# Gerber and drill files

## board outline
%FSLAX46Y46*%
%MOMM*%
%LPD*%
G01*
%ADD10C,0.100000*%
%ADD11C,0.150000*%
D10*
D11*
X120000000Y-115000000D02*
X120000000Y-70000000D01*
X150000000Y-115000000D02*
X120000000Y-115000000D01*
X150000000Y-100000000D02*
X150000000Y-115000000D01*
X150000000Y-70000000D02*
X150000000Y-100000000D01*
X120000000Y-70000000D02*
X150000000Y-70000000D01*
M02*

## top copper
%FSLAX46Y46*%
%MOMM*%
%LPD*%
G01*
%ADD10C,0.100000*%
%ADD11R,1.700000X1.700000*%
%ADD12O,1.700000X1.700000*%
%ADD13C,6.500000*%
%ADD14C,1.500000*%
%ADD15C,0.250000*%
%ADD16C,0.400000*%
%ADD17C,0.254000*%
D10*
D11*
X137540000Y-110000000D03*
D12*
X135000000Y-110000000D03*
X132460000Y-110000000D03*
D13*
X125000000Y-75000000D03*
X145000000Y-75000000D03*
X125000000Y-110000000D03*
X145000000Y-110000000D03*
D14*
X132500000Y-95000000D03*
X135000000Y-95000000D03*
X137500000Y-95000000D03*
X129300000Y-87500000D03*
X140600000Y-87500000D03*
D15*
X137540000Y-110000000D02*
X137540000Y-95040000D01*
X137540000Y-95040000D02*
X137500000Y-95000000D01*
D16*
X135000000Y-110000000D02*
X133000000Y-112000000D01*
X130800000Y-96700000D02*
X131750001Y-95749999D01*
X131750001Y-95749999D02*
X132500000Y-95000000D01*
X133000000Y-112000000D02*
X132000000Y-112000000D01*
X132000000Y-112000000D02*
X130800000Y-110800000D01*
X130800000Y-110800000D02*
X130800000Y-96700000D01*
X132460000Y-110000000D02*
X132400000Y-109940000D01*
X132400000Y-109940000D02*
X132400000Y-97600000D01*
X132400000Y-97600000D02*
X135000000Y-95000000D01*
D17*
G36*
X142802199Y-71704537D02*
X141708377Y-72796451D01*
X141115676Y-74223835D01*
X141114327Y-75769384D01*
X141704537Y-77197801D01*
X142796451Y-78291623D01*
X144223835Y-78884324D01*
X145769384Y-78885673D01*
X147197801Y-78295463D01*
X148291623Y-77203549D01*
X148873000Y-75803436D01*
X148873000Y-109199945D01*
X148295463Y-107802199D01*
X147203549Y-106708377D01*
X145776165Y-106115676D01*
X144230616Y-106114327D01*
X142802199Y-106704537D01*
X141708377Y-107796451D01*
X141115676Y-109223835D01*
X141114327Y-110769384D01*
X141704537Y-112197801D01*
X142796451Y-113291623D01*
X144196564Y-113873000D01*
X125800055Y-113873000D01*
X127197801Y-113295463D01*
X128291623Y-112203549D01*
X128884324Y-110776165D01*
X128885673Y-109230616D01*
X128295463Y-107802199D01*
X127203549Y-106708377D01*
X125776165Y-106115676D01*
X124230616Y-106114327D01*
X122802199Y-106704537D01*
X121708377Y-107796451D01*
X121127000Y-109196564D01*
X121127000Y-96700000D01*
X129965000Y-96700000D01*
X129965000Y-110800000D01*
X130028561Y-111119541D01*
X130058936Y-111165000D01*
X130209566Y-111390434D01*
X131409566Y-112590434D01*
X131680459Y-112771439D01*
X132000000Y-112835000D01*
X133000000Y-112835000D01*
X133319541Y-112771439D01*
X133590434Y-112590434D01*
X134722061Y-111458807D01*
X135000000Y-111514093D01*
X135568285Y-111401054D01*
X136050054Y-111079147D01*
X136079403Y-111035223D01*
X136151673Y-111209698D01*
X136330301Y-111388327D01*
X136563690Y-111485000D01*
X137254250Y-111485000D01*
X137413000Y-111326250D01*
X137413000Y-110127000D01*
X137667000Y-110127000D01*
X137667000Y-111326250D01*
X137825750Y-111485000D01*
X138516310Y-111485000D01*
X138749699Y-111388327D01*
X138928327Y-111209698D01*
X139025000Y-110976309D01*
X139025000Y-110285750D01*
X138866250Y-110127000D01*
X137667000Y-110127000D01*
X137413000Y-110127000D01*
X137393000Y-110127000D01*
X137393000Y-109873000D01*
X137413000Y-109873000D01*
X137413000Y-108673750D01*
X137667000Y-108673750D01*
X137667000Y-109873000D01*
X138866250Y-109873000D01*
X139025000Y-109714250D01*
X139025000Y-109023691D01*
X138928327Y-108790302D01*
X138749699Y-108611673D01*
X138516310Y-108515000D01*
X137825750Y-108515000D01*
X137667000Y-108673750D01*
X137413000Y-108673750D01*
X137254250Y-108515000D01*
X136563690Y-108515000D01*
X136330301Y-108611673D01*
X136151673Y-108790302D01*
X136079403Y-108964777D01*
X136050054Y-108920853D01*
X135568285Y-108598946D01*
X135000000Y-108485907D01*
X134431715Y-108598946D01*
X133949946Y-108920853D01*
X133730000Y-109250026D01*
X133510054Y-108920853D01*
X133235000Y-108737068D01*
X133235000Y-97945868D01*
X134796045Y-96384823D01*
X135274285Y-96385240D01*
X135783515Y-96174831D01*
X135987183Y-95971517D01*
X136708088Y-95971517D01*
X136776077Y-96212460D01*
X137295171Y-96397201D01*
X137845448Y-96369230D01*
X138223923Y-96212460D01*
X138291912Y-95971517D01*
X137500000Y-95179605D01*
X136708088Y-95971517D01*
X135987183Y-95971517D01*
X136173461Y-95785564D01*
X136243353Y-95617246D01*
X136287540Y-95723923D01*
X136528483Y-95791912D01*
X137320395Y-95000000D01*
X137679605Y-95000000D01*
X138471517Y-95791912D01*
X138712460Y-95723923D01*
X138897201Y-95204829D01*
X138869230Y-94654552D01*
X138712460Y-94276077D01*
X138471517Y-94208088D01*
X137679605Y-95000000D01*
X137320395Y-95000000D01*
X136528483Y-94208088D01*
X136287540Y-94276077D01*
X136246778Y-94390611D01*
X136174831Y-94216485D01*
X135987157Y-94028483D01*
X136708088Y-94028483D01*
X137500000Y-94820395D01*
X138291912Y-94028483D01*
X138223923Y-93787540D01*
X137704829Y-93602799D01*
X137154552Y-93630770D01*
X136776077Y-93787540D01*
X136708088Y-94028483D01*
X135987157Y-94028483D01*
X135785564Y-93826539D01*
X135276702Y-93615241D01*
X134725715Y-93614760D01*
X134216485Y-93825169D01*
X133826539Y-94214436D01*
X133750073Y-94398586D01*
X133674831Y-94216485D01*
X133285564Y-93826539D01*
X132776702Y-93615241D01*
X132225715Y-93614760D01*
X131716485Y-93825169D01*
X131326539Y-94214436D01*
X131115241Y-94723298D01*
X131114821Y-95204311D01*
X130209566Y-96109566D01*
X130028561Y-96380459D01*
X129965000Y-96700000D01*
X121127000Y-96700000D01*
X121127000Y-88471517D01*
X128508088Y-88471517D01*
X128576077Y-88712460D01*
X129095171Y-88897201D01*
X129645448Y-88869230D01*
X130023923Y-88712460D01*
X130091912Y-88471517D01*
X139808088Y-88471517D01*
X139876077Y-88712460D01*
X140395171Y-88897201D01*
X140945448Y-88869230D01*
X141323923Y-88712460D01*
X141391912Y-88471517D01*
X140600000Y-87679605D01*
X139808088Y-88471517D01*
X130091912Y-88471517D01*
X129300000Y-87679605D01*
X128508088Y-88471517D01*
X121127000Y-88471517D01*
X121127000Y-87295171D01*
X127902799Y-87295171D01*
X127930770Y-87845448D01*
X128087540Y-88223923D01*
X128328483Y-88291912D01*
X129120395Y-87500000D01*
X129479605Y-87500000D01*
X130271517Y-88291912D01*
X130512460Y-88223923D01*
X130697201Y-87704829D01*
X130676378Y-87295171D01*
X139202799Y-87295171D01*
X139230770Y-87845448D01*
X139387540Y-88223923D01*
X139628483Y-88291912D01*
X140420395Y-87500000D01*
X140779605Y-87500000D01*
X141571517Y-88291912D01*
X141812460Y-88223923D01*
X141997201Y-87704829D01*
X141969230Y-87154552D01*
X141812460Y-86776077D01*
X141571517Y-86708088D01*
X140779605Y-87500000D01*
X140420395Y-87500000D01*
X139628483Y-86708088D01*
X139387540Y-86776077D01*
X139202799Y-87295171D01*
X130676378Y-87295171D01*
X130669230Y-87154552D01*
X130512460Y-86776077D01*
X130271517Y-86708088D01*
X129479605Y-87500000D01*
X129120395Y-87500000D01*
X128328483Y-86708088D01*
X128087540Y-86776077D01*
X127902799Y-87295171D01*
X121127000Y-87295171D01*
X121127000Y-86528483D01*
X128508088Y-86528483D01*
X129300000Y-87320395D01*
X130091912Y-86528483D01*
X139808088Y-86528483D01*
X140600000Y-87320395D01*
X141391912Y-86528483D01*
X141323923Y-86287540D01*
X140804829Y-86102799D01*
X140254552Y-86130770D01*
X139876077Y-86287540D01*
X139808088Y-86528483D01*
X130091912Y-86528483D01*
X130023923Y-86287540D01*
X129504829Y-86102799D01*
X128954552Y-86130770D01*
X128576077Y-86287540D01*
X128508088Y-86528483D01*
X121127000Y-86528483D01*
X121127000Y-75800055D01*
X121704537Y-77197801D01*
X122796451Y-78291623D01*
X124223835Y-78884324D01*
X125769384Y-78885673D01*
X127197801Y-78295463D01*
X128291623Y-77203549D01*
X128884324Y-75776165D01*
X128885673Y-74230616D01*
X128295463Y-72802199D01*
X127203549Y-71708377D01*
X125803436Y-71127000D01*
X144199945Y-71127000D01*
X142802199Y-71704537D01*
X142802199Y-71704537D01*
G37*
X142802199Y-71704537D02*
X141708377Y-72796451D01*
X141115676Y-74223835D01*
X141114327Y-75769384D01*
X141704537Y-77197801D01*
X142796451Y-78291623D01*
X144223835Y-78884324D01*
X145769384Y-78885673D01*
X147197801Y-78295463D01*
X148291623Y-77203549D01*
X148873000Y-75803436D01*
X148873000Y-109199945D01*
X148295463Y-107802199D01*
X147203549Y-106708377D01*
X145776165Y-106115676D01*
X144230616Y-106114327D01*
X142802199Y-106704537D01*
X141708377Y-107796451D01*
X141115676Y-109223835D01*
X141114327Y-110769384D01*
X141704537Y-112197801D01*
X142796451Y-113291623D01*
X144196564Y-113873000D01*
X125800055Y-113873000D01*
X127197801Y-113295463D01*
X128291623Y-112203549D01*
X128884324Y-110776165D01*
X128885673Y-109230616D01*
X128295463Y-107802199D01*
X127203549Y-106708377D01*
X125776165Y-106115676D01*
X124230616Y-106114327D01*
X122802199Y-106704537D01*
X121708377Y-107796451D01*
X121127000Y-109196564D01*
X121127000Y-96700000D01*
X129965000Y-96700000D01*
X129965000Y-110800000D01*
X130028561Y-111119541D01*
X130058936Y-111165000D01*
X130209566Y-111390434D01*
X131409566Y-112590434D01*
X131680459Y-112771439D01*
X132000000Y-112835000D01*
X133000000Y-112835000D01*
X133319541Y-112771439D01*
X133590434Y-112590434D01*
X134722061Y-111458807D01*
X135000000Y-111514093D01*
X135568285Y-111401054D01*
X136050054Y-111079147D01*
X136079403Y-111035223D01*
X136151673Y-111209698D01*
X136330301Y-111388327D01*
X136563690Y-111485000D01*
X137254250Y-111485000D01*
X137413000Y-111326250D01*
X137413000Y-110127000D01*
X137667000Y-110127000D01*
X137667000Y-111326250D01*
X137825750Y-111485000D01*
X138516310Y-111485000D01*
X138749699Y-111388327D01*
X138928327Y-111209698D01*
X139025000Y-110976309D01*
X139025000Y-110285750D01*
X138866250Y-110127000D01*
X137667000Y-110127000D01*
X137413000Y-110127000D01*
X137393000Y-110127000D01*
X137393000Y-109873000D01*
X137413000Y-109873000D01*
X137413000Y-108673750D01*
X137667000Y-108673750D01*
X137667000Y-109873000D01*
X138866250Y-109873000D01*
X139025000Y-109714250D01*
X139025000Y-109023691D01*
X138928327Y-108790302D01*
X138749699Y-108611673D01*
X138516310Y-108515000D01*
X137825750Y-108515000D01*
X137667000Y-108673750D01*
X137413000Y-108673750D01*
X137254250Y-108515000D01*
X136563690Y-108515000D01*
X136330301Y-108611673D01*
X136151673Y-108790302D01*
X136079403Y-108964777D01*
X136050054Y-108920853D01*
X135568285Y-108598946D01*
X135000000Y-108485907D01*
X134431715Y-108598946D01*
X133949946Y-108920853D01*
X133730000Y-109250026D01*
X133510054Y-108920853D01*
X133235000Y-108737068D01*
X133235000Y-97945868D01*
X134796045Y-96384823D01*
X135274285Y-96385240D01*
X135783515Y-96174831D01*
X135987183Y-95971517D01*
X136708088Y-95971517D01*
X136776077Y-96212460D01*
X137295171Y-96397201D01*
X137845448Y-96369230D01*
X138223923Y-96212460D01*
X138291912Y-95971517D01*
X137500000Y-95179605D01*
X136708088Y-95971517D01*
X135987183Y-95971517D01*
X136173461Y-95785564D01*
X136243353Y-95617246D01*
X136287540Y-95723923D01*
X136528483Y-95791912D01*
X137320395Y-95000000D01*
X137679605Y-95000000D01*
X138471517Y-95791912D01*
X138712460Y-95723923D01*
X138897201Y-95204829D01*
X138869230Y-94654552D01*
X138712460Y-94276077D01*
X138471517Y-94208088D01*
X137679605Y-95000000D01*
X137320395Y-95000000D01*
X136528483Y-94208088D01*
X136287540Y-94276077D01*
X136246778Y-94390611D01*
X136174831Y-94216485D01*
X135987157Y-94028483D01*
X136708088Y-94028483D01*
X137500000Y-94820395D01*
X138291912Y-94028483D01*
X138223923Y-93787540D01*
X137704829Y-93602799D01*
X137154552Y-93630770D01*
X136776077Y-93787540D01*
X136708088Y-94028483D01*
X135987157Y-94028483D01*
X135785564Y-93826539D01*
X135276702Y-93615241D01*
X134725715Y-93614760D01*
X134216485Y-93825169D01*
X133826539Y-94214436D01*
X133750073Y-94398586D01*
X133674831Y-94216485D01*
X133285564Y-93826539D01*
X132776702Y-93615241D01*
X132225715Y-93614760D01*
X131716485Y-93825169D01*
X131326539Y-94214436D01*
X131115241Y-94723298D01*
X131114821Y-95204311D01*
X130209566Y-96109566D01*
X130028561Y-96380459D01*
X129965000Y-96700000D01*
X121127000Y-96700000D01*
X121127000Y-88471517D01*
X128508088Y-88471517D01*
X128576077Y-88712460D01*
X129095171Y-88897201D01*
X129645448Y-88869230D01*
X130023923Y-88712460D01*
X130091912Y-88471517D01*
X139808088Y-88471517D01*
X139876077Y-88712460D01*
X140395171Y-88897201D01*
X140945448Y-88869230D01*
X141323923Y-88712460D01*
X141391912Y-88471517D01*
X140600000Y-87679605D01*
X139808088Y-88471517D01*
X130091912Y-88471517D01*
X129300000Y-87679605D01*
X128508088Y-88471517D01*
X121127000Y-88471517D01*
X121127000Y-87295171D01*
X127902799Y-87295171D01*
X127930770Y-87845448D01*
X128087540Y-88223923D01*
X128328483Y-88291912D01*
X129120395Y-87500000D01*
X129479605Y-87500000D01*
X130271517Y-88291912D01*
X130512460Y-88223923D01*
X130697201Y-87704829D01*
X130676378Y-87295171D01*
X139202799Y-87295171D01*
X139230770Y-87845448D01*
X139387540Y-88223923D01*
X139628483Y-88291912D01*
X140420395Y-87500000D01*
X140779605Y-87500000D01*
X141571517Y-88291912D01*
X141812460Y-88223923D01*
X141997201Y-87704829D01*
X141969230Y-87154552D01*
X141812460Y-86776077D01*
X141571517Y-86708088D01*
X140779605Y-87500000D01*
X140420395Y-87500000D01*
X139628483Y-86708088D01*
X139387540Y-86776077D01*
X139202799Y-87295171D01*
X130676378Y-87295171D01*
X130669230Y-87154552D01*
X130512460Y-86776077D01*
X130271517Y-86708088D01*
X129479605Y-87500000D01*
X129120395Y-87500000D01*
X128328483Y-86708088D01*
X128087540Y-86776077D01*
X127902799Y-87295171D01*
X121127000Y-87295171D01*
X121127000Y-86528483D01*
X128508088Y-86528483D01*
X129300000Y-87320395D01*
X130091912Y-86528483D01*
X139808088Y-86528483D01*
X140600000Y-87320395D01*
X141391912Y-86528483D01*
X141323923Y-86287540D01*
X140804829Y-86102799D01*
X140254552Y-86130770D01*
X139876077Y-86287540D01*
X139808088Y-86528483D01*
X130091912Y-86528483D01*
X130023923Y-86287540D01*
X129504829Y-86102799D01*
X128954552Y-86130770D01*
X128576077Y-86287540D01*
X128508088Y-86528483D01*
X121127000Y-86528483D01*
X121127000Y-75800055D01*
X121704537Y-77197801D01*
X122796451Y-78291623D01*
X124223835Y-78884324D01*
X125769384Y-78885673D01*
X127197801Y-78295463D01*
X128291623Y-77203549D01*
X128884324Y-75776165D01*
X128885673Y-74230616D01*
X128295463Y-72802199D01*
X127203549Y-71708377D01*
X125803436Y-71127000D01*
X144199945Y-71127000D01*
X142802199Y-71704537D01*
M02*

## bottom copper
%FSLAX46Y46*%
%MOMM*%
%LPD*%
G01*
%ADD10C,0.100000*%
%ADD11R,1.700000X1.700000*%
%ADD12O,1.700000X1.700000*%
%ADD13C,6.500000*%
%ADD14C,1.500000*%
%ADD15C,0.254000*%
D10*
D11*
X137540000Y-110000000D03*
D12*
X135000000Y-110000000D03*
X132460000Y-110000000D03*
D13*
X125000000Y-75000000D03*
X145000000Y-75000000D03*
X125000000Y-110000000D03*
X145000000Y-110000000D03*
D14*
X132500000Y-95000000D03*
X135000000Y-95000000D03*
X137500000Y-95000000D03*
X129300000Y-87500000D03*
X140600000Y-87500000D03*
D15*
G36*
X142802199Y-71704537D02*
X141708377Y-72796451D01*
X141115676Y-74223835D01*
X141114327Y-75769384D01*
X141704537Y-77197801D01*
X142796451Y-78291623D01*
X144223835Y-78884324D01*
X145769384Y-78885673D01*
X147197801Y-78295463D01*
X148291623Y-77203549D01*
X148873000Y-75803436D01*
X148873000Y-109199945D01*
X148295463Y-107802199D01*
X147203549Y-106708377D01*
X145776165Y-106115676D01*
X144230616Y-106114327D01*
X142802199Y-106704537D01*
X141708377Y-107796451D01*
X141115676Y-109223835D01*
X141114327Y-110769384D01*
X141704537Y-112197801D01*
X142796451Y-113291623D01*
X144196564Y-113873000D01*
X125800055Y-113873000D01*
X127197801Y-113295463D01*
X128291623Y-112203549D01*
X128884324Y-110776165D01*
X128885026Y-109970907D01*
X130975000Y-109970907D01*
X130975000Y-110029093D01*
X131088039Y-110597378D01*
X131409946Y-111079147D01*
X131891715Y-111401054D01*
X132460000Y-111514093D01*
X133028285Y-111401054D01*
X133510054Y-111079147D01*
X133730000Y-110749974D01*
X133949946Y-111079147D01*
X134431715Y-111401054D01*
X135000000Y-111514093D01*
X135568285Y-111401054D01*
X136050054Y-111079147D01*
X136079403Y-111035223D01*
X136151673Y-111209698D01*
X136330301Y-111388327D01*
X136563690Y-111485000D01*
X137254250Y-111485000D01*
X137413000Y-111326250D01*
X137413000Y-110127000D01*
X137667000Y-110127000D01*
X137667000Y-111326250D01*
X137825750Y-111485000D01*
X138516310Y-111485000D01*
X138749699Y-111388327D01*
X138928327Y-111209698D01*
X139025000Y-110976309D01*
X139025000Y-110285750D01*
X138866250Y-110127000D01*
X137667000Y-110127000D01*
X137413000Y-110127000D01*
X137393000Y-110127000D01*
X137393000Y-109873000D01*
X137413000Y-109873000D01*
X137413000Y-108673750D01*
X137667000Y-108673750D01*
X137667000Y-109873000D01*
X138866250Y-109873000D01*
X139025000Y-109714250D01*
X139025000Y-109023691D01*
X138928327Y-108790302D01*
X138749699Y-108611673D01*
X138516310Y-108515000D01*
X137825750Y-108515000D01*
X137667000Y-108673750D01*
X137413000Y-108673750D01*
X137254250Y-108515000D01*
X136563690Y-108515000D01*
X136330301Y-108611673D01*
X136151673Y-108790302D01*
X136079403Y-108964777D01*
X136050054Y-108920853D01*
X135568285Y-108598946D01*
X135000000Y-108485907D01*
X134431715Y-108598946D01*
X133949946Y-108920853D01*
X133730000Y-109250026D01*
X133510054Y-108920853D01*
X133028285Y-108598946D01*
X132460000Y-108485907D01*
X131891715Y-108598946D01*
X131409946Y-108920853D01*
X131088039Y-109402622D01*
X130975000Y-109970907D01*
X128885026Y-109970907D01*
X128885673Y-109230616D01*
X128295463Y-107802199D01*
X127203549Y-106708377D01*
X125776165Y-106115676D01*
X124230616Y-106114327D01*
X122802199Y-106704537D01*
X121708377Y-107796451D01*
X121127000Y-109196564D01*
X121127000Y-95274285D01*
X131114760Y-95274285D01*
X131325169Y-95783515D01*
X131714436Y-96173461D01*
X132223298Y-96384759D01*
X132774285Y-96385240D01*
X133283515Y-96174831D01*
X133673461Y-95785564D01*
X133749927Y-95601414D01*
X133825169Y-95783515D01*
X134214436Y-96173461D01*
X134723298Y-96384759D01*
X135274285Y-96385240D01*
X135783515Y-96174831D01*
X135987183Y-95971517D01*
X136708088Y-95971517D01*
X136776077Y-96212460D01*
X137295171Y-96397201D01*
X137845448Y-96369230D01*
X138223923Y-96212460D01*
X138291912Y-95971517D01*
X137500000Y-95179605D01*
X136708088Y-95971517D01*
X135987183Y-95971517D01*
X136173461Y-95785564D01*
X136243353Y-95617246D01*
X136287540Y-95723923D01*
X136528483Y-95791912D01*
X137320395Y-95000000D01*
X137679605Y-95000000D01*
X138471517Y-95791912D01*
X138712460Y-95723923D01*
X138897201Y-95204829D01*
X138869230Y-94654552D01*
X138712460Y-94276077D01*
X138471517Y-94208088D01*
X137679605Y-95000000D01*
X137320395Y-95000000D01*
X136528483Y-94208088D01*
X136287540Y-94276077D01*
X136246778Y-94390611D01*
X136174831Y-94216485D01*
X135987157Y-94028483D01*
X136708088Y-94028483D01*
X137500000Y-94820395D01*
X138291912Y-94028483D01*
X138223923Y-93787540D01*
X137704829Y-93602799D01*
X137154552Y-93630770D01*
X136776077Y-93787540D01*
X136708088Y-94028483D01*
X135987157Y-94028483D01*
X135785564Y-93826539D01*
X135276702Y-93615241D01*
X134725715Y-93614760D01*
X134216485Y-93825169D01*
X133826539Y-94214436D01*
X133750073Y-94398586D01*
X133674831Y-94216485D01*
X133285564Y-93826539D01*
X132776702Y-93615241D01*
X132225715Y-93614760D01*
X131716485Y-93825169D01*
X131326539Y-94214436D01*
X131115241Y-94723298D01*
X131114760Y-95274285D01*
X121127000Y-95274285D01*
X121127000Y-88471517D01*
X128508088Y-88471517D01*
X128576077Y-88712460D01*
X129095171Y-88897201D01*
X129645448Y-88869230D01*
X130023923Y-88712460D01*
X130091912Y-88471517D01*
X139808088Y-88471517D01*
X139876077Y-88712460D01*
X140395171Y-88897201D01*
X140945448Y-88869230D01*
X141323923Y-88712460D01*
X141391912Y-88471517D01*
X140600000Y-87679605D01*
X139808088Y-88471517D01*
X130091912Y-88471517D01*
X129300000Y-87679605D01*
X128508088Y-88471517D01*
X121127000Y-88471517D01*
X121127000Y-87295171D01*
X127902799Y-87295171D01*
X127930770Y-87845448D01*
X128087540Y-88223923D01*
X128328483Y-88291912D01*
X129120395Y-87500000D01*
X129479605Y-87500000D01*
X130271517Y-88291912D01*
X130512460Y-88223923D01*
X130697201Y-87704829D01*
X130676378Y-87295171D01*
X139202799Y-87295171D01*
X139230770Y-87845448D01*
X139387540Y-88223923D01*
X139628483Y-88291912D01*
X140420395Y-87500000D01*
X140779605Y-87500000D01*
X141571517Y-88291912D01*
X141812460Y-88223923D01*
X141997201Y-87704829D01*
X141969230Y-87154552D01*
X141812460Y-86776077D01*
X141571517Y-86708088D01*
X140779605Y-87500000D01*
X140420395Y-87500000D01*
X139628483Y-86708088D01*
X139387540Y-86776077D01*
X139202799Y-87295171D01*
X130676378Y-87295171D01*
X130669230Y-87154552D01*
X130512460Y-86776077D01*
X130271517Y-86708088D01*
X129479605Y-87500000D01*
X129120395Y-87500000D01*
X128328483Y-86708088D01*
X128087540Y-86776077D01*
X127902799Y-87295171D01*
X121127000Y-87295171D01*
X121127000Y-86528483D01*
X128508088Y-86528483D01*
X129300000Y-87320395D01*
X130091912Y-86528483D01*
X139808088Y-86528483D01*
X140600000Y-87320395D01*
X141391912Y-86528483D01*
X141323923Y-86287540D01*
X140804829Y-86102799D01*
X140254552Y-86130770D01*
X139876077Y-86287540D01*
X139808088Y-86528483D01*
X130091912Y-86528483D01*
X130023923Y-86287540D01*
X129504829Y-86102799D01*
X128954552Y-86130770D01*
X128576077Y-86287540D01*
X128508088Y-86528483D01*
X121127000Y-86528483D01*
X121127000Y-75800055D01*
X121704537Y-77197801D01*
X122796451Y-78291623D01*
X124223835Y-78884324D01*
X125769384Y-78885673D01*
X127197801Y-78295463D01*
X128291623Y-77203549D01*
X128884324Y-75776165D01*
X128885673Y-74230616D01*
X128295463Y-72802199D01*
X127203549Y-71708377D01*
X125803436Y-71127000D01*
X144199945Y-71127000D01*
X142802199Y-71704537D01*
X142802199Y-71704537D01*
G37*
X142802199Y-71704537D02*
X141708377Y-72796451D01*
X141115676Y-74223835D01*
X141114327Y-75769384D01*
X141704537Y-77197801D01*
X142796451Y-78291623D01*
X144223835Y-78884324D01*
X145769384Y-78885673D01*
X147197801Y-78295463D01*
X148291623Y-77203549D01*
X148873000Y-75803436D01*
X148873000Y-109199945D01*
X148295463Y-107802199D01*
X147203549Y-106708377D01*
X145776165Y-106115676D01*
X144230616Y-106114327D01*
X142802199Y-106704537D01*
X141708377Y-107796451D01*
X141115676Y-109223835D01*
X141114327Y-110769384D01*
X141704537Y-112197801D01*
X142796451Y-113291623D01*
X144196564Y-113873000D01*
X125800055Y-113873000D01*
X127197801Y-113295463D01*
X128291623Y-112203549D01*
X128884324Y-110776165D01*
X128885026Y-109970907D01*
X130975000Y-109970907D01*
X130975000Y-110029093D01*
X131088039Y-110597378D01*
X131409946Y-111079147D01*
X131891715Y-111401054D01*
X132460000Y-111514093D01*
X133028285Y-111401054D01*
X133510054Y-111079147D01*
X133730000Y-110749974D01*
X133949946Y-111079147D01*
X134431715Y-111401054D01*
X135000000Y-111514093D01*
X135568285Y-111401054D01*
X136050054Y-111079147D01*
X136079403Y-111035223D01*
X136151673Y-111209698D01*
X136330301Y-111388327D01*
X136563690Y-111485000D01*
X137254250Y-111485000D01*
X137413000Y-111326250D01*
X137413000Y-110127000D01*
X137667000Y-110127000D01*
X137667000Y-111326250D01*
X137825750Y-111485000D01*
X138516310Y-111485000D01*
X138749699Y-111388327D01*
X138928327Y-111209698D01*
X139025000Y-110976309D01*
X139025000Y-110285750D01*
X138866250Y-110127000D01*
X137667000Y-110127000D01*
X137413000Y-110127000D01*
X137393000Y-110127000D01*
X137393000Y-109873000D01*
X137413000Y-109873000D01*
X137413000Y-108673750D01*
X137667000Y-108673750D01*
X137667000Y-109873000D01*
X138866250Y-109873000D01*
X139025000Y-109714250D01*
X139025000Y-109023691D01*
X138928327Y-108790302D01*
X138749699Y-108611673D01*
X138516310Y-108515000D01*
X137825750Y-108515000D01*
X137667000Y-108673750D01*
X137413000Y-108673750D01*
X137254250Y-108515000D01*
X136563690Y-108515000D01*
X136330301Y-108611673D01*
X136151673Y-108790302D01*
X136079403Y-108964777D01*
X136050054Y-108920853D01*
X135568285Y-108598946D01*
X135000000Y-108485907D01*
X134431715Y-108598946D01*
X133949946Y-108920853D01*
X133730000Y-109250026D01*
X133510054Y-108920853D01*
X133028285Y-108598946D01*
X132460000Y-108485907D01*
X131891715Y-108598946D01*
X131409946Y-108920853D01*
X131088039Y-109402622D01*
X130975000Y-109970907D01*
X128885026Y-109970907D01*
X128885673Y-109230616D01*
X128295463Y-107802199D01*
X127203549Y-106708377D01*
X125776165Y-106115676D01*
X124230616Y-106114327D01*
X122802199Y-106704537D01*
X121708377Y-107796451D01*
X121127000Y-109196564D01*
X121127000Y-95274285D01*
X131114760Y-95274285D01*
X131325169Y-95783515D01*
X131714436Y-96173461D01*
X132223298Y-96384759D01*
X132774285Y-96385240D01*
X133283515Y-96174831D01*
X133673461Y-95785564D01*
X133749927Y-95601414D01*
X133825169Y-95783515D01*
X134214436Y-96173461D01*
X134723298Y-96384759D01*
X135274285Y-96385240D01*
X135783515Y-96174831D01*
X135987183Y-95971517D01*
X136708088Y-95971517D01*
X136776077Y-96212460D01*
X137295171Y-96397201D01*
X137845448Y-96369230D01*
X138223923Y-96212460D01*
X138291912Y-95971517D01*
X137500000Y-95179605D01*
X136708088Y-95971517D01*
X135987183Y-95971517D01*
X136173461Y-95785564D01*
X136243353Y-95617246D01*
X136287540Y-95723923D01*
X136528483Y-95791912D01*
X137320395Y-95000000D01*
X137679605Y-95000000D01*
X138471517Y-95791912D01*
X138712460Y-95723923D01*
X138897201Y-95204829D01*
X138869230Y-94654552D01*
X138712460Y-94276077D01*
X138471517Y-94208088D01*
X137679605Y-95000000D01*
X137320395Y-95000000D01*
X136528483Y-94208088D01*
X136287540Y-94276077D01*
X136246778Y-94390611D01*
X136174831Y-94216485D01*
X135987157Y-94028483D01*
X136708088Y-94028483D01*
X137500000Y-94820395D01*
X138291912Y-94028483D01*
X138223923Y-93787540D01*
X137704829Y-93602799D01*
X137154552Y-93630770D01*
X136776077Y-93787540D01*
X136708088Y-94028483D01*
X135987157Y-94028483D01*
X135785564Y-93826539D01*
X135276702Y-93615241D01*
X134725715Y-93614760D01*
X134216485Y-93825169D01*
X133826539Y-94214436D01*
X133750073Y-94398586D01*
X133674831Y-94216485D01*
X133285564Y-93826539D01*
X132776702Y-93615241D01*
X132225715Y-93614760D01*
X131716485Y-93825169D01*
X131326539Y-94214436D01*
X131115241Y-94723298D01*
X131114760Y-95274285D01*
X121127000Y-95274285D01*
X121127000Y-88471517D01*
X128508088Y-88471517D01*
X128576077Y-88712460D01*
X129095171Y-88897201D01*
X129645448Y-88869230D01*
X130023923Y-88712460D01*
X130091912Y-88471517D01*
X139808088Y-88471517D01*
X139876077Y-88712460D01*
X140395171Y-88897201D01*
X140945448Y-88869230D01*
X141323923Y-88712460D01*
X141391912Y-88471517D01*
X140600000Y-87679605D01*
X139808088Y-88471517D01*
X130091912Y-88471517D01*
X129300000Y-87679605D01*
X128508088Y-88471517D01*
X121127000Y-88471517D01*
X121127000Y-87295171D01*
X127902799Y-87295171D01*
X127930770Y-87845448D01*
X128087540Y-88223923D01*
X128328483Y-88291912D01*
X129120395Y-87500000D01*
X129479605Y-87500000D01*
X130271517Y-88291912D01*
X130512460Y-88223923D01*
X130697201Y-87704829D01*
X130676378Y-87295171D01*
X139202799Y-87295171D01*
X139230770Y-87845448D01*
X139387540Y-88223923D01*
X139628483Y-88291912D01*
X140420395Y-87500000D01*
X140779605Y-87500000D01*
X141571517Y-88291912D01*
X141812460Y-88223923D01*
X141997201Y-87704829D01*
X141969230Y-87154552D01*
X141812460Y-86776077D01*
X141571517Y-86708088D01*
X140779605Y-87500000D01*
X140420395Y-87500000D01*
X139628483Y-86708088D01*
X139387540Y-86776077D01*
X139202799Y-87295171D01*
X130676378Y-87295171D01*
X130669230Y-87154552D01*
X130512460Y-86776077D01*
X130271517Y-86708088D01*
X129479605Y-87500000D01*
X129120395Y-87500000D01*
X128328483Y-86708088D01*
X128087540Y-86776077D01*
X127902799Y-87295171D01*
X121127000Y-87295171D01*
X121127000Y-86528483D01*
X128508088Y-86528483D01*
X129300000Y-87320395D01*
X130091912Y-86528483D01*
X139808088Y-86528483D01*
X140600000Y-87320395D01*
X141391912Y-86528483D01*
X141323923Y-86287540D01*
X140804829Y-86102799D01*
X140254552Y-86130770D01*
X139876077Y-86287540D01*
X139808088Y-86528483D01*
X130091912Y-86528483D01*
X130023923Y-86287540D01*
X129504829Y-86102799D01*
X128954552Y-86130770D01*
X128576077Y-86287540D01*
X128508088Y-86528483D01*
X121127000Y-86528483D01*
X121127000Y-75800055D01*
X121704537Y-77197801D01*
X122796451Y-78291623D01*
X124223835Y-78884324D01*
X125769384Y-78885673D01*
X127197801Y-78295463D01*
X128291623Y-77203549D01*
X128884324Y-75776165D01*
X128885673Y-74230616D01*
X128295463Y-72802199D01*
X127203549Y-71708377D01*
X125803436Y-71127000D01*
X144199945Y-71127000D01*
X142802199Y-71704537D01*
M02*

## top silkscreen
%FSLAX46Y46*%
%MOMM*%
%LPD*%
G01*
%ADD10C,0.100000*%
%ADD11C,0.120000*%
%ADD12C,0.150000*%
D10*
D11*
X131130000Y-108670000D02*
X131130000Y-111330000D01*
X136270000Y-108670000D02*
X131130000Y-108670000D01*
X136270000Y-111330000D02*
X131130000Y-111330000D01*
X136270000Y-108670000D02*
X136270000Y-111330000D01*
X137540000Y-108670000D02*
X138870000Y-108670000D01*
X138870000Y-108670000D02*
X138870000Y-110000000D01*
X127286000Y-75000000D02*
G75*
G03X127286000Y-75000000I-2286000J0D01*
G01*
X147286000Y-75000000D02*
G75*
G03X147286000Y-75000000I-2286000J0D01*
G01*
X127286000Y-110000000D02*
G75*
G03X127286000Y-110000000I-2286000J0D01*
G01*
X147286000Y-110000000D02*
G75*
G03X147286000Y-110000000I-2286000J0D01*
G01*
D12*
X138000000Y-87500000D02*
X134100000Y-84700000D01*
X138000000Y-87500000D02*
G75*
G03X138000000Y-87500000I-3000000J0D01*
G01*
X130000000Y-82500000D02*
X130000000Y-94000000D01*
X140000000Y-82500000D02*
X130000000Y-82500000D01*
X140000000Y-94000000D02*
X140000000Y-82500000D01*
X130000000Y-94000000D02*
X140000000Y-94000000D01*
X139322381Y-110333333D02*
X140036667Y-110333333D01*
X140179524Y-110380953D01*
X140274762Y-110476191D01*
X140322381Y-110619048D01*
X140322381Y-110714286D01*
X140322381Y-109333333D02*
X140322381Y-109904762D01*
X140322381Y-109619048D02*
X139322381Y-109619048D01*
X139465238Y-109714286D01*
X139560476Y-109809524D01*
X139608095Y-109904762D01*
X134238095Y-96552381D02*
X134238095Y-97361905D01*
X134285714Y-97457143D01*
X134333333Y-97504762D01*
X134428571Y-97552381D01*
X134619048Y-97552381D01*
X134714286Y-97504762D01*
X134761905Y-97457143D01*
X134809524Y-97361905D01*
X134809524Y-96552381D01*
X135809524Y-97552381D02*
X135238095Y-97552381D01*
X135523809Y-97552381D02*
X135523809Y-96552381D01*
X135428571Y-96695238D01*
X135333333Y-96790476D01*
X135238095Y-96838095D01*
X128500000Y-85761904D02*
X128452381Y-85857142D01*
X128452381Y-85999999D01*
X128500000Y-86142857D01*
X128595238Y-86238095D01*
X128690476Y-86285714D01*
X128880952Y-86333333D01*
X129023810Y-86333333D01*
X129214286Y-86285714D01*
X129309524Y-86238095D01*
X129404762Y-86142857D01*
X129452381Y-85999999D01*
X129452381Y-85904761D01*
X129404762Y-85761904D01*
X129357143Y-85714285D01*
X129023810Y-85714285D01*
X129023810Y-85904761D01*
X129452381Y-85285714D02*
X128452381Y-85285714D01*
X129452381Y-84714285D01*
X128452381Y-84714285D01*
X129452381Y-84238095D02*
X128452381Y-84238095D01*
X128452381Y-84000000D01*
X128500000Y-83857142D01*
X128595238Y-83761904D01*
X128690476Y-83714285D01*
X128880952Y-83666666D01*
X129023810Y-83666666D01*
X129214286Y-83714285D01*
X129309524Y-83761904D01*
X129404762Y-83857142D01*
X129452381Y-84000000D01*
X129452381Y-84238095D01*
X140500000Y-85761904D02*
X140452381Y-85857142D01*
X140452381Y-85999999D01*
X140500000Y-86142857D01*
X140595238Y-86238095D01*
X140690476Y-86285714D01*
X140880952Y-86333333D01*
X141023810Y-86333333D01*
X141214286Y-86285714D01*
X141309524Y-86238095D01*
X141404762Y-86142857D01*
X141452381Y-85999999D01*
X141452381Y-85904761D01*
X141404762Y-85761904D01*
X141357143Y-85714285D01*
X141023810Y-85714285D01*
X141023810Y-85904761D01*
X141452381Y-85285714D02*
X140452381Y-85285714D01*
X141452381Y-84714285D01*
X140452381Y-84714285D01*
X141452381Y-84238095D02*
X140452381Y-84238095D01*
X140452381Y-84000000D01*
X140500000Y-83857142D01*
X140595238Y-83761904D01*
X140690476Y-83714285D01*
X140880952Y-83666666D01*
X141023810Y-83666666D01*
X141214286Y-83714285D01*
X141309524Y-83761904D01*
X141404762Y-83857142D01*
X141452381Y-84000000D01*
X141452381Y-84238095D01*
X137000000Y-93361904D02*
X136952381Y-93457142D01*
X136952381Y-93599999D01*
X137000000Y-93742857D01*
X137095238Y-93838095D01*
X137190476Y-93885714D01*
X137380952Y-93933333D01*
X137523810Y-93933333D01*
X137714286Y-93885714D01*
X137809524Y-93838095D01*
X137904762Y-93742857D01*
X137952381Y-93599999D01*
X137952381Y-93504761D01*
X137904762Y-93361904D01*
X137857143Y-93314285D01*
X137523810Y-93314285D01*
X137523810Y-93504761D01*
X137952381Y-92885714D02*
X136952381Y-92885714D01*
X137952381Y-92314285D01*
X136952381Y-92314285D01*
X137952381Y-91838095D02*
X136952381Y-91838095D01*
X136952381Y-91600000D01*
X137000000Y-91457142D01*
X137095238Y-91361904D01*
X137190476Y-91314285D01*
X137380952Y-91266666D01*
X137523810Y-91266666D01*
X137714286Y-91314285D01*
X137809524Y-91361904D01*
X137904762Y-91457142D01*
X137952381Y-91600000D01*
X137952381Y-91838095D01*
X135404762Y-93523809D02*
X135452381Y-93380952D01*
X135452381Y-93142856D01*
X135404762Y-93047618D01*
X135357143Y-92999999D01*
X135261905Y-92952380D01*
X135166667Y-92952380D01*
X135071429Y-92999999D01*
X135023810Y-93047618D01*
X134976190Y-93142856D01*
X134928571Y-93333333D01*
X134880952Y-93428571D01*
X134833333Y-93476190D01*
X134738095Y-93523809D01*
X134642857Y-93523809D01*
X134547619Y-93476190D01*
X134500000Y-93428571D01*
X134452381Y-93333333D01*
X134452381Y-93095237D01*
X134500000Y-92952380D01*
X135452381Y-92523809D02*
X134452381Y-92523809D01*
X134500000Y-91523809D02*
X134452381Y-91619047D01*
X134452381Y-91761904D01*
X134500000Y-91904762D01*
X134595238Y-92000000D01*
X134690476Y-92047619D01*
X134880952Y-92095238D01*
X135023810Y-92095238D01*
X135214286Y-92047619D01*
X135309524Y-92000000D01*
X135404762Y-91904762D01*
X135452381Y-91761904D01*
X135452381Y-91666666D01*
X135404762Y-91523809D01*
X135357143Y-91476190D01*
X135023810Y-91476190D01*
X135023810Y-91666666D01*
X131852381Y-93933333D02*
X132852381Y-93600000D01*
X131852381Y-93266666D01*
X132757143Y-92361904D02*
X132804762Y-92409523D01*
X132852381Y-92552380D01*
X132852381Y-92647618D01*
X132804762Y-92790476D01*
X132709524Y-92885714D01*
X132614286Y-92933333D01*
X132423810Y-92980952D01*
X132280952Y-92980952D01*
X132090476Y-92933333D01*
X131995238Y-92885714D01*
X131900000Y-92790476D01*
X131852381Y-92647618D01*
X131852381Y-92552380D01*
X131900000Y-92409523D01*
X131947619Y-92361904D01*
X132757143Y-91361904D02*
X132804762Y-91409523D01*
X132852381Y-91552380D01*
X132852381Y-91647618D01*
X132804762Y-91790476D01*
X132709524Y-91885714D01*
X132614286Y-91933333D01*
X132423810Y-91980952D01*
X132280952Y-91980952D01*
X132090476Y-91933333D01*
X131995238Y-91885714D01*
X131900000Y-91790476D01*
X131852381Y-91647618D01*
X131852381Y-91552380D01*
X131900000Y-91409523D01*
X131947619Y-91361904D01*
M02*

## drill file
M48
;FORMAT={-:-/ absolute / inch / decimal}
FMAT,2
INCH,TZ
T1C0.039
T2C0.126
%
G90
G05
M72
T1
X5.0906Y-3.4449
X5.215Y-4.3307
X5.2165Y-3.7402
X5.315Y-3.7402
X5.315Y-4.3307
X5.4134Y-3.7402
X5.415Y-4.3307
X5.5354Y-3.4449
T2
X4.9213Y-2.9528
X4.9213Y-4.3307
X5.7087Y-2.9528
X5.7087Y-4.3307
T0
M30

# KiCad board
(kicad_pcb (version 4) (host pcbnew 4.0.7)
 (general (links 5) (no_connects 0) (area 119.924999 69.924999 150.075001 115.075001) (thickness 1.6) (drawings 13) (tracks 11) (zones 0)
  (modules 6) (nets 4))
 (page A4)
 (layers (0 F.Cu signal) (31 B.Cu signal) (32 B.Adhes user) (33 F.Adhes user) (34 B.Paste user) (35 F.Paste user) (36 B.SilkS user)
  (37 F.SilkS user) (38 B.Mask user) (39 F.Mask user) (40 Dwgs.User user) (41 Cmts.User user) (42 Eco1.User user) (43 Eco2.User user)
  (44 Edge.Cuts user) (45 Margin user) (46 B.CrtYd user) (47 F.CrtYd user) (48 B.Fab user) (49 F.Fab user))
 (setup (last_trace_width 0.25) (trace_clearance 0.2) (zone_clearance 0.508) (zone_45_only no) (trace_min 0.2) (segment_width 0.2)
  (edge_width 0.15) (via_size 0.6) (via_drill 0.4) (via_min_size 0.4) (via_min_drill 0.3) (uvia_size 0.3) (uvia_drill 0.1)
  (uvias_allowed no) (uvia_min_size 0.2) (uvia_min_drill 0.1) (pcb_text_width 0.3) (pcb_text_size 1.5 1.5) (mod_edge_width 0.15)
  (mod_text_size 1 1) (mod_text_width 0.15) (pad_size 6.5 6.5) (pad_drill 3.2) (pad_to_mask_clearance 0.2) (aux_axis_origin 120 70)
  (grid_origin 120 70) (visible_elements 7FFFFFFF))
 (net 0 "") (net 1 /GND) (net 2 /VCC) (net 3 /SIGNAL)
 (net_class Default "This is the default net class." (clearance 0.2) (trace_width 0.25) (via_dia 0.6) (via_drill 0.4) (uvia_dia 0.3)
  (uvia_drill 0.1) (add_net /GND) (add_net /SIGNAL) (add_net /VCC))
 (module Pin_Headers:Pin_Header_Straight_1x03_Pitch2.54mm (layer F.Cu) (at 137.54 110 270)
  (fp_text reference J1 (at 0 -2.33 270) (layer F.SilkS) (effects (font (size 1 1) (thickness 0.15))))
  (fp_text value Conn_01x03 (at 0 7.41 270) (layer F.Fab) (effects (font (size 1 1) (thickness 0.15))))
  (fp_line (start -1.33 6.41) (end 1.33 6.41) (layer F.SilkS) (width 0.12))
  (fp_line (start -1.33 1.27) (end -1.33 6.41) (layer F.SilkS) (width 0.12))
  (fp_line (start 1.33 1.27) (end 1.33 6.41) (layer F.SilkS) (width 0.12))
  (fp_line (start -1.33 1.27) (end 1.33 1.27) (layer F.SilkS) (width 0.12))
  (fp_line (start -1.33 0) (end -1.33 -1.33) (layer F.SilkS) (width 0.12))
  (fp_line (start -1.33 -1.33) (end 0 -1.33) (layer F.SilkS) (width 0.12))
  (pad 1 thru_hole rect (at 0 0 270) (size 1.7 1.7) (drill 1) (layers *.Cu *.Mask) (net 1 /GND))
  (pad 2 thru_hole oval (at 0 2.54 270) (size 1.7 1.7) (drill 1) (layers *.Cu *.Mask) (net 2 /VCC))
  (pad 3 thru_hole oval (at 0 5.08 270) (size 1.7 1.7) (drill 1) (layers *.Cu *.Mask) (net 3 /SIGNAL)))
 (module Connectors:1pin (layer F.Cu) (at 125 75)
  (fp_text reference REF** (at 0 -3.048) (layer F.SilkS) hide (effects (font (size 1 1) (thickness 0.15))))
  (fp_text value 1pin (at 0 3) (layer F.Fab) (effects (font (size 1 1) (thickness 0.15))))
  (fp_circle (center 0 0) (end 0 -2.286) (layer F.SilkS) (width 0.12))
  (pad ~ thru_hole circle (at 0 0) (size 6.5 6.5) (drill 3.2) (layers *.Cu *.Mask)))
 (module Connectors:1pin (layer F.Cu) (at 145 75)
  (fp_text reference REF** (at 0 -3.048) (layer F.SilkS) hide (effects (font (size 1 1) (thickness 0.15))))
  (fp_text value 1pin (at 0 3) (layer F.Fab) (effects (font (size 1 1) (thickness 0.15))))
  (fp_circle (center 0 0) (end 0 -2.286) (layer F.SilkS) (width 0.12))
  (pad ~ thru_hole circle (at 0 0) (size 6.5 6.5) (drill 3.2) (layers *.Cu *.Mask)))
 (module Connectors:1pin (layer F.Cu) (at 125 110)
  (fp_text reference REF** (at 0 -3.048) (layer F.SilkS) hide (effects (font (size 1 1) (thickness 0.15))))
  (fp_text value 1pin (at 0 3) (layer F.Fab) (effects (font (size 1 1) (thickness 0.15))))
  (fp_circle (center 0 0) (end 0 -2.286) (layer F.SilkS) (width 0.12))
  (pad ~ thru_hole circle (at 0 0) (size 6.5 6.5) (drill 3.2) (layers *.Cu *.Mask)))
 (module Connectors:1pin (layer F.Cu) (at 145 110)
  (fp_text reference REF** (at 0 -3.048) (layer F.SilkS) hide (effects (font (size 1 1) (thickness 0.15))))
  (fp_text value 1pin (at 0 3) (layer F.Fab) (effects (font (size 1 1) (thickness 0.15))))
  (fp_circle (center 0 0) (end 0 -2.286) (layer F.SilkS) (width 0.12))
  (pad ~ thru_hole circle (at 0 0) (size 6.5 6.5) (drill 3.2) (layers *.Cu *.Mask)))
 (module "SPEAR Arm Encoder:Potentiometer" (layer F.Cu) (at 135 90)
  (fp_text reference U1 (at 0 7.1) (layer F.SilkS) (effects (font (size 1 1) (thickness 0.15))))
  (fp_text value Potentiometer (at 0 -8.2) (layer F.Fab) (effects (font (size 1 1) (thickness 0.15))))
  (fp_line (start 3 -2.5) (end -0.9 -5.3) (layer F.SilkS) (width 0.15))
  (fp_circle (center 0 -2.5) (end 3 -2.5) (layer F.SilkS) (width 0.15))
  (fp_line (start -5 -7.5) (end -5 4) (layer F.SilkS) (width 0.15))
  (fp_line (start 5 -7.5) (end -5 -7.5) (layer F.SilkS) (width 0.15))
  (fp_line (start 5 4) (end 5 -7.5) (layer F.SilkS) (width 0.15))
  (fp_line (start -5 4) (end 5 4) (layer F.SilkS) (width 0.15))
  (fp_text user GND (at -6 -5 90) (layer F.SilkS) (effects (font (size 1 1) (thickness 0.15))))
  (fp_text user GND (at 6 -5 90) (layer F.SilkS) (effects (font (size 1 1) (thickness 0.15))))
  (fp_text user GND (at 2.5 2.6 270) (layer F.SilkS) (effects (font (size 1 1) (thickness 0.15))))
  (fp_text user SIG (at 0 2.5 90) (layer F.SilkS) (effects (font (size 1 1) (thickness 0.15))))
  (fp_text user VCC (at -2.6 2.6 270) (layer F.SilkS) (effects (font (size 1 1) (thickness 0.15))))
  (pad 1 thru_hole circle (at -2.5 5) (size 1.5 1.5) (drill 1) (layers *.Cu *.Mask) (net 2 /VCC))
  (pad 2 thru_hole circle (at 0 5) (size 1.5 1.5) (drill 1) (layers *.Cu *.Mask) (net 3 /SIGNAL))
  (pad 3 thru_hole circle (at 2.5 5) (size 1.5 1.5) (drill 1) (layers *.Cu *.Mask) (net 1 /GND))
  (pad 4 thru_hole circle (at -5.7 -2.5) (size 1.5 1.5) (drill 1) (layers *.Cu *.Mask) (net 1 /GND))
  (pad 5 thru_hole circle (at 5.6 -2.5) (size 1.5 1.5) (drill 1) (layers *.Cu *.Mask) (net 1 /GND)))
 (gr_line (start 120 115) (end 120 70) (layer Edge.Cuts) (width 0.15))
 (gr_line (start 150 115) (end 120 115) (layer Edge.Cuts) (width 0.15))
 (gr_line (start 150 100) (end 150 115) (layer Edge.Cuts) (width 0.15))
 (gr_line (start 150 70) (end 150 100) (layer Edge.Cuts) (width 0.15))
 (gr_line (start 120 70) (end 150 70) (layer Edge.Cuts) (width 0.15))
 (segment (start 137.54 110) (end 137.54 95.04) (width 0.25) (layer F.Cu) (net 1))
 (segment (start 137.54 95.04) (end 137.5 95) (width 0.25) (layer F.Cu) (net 1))
 (segment (start 135 110) (end 133 112) (width 0.4) (layer F.Cu) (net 2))
 (segment (start 130.8 96.7) (end 131.750001 95.749999) (width 0.4) (layer F.Cu) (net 2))
 (segment (start 131.750001 95.749999) (end 132.5 95) (width 0.4) (layer F.Cu) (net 2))
 (segment (start 133 112) (end 132 112) (width 0.4) (layer F.Cu) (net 2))
 (segment (start 132 112) (end 130.8 110.8) (width 0.4) (layer F.Cu) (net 2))
 (segment (start 130.8 110.8) (end 130.8 96.7) (width 0.4) (layer F.Cu) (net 2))
 (segment (start 132.46 110) (end 132.4 109.94) (width 0.4) (layer F.Cu) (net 3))
 (segment (start 132.4 109.94) (end 132.4 97.6) (width 0.4) (layer F.Cu) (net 3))
 (segment (start 132.4 97.6) (end 135 95) (width 0.4) (layer F.Cu) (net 3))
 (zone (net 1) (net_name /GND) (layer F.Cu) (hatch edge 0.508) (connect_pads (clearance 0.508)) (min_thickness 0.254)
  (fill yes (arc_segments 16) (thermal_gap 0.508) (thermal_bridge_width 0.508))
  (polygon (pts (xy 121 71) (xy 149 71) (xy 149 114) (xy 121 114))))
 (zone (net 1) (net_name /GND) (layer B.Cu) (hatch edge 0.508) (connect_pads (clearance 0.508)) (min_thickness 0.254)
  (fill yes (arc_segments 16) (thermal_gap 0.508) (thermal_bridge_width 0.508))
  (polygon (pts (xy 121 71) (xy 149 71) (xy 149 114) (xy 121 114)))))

